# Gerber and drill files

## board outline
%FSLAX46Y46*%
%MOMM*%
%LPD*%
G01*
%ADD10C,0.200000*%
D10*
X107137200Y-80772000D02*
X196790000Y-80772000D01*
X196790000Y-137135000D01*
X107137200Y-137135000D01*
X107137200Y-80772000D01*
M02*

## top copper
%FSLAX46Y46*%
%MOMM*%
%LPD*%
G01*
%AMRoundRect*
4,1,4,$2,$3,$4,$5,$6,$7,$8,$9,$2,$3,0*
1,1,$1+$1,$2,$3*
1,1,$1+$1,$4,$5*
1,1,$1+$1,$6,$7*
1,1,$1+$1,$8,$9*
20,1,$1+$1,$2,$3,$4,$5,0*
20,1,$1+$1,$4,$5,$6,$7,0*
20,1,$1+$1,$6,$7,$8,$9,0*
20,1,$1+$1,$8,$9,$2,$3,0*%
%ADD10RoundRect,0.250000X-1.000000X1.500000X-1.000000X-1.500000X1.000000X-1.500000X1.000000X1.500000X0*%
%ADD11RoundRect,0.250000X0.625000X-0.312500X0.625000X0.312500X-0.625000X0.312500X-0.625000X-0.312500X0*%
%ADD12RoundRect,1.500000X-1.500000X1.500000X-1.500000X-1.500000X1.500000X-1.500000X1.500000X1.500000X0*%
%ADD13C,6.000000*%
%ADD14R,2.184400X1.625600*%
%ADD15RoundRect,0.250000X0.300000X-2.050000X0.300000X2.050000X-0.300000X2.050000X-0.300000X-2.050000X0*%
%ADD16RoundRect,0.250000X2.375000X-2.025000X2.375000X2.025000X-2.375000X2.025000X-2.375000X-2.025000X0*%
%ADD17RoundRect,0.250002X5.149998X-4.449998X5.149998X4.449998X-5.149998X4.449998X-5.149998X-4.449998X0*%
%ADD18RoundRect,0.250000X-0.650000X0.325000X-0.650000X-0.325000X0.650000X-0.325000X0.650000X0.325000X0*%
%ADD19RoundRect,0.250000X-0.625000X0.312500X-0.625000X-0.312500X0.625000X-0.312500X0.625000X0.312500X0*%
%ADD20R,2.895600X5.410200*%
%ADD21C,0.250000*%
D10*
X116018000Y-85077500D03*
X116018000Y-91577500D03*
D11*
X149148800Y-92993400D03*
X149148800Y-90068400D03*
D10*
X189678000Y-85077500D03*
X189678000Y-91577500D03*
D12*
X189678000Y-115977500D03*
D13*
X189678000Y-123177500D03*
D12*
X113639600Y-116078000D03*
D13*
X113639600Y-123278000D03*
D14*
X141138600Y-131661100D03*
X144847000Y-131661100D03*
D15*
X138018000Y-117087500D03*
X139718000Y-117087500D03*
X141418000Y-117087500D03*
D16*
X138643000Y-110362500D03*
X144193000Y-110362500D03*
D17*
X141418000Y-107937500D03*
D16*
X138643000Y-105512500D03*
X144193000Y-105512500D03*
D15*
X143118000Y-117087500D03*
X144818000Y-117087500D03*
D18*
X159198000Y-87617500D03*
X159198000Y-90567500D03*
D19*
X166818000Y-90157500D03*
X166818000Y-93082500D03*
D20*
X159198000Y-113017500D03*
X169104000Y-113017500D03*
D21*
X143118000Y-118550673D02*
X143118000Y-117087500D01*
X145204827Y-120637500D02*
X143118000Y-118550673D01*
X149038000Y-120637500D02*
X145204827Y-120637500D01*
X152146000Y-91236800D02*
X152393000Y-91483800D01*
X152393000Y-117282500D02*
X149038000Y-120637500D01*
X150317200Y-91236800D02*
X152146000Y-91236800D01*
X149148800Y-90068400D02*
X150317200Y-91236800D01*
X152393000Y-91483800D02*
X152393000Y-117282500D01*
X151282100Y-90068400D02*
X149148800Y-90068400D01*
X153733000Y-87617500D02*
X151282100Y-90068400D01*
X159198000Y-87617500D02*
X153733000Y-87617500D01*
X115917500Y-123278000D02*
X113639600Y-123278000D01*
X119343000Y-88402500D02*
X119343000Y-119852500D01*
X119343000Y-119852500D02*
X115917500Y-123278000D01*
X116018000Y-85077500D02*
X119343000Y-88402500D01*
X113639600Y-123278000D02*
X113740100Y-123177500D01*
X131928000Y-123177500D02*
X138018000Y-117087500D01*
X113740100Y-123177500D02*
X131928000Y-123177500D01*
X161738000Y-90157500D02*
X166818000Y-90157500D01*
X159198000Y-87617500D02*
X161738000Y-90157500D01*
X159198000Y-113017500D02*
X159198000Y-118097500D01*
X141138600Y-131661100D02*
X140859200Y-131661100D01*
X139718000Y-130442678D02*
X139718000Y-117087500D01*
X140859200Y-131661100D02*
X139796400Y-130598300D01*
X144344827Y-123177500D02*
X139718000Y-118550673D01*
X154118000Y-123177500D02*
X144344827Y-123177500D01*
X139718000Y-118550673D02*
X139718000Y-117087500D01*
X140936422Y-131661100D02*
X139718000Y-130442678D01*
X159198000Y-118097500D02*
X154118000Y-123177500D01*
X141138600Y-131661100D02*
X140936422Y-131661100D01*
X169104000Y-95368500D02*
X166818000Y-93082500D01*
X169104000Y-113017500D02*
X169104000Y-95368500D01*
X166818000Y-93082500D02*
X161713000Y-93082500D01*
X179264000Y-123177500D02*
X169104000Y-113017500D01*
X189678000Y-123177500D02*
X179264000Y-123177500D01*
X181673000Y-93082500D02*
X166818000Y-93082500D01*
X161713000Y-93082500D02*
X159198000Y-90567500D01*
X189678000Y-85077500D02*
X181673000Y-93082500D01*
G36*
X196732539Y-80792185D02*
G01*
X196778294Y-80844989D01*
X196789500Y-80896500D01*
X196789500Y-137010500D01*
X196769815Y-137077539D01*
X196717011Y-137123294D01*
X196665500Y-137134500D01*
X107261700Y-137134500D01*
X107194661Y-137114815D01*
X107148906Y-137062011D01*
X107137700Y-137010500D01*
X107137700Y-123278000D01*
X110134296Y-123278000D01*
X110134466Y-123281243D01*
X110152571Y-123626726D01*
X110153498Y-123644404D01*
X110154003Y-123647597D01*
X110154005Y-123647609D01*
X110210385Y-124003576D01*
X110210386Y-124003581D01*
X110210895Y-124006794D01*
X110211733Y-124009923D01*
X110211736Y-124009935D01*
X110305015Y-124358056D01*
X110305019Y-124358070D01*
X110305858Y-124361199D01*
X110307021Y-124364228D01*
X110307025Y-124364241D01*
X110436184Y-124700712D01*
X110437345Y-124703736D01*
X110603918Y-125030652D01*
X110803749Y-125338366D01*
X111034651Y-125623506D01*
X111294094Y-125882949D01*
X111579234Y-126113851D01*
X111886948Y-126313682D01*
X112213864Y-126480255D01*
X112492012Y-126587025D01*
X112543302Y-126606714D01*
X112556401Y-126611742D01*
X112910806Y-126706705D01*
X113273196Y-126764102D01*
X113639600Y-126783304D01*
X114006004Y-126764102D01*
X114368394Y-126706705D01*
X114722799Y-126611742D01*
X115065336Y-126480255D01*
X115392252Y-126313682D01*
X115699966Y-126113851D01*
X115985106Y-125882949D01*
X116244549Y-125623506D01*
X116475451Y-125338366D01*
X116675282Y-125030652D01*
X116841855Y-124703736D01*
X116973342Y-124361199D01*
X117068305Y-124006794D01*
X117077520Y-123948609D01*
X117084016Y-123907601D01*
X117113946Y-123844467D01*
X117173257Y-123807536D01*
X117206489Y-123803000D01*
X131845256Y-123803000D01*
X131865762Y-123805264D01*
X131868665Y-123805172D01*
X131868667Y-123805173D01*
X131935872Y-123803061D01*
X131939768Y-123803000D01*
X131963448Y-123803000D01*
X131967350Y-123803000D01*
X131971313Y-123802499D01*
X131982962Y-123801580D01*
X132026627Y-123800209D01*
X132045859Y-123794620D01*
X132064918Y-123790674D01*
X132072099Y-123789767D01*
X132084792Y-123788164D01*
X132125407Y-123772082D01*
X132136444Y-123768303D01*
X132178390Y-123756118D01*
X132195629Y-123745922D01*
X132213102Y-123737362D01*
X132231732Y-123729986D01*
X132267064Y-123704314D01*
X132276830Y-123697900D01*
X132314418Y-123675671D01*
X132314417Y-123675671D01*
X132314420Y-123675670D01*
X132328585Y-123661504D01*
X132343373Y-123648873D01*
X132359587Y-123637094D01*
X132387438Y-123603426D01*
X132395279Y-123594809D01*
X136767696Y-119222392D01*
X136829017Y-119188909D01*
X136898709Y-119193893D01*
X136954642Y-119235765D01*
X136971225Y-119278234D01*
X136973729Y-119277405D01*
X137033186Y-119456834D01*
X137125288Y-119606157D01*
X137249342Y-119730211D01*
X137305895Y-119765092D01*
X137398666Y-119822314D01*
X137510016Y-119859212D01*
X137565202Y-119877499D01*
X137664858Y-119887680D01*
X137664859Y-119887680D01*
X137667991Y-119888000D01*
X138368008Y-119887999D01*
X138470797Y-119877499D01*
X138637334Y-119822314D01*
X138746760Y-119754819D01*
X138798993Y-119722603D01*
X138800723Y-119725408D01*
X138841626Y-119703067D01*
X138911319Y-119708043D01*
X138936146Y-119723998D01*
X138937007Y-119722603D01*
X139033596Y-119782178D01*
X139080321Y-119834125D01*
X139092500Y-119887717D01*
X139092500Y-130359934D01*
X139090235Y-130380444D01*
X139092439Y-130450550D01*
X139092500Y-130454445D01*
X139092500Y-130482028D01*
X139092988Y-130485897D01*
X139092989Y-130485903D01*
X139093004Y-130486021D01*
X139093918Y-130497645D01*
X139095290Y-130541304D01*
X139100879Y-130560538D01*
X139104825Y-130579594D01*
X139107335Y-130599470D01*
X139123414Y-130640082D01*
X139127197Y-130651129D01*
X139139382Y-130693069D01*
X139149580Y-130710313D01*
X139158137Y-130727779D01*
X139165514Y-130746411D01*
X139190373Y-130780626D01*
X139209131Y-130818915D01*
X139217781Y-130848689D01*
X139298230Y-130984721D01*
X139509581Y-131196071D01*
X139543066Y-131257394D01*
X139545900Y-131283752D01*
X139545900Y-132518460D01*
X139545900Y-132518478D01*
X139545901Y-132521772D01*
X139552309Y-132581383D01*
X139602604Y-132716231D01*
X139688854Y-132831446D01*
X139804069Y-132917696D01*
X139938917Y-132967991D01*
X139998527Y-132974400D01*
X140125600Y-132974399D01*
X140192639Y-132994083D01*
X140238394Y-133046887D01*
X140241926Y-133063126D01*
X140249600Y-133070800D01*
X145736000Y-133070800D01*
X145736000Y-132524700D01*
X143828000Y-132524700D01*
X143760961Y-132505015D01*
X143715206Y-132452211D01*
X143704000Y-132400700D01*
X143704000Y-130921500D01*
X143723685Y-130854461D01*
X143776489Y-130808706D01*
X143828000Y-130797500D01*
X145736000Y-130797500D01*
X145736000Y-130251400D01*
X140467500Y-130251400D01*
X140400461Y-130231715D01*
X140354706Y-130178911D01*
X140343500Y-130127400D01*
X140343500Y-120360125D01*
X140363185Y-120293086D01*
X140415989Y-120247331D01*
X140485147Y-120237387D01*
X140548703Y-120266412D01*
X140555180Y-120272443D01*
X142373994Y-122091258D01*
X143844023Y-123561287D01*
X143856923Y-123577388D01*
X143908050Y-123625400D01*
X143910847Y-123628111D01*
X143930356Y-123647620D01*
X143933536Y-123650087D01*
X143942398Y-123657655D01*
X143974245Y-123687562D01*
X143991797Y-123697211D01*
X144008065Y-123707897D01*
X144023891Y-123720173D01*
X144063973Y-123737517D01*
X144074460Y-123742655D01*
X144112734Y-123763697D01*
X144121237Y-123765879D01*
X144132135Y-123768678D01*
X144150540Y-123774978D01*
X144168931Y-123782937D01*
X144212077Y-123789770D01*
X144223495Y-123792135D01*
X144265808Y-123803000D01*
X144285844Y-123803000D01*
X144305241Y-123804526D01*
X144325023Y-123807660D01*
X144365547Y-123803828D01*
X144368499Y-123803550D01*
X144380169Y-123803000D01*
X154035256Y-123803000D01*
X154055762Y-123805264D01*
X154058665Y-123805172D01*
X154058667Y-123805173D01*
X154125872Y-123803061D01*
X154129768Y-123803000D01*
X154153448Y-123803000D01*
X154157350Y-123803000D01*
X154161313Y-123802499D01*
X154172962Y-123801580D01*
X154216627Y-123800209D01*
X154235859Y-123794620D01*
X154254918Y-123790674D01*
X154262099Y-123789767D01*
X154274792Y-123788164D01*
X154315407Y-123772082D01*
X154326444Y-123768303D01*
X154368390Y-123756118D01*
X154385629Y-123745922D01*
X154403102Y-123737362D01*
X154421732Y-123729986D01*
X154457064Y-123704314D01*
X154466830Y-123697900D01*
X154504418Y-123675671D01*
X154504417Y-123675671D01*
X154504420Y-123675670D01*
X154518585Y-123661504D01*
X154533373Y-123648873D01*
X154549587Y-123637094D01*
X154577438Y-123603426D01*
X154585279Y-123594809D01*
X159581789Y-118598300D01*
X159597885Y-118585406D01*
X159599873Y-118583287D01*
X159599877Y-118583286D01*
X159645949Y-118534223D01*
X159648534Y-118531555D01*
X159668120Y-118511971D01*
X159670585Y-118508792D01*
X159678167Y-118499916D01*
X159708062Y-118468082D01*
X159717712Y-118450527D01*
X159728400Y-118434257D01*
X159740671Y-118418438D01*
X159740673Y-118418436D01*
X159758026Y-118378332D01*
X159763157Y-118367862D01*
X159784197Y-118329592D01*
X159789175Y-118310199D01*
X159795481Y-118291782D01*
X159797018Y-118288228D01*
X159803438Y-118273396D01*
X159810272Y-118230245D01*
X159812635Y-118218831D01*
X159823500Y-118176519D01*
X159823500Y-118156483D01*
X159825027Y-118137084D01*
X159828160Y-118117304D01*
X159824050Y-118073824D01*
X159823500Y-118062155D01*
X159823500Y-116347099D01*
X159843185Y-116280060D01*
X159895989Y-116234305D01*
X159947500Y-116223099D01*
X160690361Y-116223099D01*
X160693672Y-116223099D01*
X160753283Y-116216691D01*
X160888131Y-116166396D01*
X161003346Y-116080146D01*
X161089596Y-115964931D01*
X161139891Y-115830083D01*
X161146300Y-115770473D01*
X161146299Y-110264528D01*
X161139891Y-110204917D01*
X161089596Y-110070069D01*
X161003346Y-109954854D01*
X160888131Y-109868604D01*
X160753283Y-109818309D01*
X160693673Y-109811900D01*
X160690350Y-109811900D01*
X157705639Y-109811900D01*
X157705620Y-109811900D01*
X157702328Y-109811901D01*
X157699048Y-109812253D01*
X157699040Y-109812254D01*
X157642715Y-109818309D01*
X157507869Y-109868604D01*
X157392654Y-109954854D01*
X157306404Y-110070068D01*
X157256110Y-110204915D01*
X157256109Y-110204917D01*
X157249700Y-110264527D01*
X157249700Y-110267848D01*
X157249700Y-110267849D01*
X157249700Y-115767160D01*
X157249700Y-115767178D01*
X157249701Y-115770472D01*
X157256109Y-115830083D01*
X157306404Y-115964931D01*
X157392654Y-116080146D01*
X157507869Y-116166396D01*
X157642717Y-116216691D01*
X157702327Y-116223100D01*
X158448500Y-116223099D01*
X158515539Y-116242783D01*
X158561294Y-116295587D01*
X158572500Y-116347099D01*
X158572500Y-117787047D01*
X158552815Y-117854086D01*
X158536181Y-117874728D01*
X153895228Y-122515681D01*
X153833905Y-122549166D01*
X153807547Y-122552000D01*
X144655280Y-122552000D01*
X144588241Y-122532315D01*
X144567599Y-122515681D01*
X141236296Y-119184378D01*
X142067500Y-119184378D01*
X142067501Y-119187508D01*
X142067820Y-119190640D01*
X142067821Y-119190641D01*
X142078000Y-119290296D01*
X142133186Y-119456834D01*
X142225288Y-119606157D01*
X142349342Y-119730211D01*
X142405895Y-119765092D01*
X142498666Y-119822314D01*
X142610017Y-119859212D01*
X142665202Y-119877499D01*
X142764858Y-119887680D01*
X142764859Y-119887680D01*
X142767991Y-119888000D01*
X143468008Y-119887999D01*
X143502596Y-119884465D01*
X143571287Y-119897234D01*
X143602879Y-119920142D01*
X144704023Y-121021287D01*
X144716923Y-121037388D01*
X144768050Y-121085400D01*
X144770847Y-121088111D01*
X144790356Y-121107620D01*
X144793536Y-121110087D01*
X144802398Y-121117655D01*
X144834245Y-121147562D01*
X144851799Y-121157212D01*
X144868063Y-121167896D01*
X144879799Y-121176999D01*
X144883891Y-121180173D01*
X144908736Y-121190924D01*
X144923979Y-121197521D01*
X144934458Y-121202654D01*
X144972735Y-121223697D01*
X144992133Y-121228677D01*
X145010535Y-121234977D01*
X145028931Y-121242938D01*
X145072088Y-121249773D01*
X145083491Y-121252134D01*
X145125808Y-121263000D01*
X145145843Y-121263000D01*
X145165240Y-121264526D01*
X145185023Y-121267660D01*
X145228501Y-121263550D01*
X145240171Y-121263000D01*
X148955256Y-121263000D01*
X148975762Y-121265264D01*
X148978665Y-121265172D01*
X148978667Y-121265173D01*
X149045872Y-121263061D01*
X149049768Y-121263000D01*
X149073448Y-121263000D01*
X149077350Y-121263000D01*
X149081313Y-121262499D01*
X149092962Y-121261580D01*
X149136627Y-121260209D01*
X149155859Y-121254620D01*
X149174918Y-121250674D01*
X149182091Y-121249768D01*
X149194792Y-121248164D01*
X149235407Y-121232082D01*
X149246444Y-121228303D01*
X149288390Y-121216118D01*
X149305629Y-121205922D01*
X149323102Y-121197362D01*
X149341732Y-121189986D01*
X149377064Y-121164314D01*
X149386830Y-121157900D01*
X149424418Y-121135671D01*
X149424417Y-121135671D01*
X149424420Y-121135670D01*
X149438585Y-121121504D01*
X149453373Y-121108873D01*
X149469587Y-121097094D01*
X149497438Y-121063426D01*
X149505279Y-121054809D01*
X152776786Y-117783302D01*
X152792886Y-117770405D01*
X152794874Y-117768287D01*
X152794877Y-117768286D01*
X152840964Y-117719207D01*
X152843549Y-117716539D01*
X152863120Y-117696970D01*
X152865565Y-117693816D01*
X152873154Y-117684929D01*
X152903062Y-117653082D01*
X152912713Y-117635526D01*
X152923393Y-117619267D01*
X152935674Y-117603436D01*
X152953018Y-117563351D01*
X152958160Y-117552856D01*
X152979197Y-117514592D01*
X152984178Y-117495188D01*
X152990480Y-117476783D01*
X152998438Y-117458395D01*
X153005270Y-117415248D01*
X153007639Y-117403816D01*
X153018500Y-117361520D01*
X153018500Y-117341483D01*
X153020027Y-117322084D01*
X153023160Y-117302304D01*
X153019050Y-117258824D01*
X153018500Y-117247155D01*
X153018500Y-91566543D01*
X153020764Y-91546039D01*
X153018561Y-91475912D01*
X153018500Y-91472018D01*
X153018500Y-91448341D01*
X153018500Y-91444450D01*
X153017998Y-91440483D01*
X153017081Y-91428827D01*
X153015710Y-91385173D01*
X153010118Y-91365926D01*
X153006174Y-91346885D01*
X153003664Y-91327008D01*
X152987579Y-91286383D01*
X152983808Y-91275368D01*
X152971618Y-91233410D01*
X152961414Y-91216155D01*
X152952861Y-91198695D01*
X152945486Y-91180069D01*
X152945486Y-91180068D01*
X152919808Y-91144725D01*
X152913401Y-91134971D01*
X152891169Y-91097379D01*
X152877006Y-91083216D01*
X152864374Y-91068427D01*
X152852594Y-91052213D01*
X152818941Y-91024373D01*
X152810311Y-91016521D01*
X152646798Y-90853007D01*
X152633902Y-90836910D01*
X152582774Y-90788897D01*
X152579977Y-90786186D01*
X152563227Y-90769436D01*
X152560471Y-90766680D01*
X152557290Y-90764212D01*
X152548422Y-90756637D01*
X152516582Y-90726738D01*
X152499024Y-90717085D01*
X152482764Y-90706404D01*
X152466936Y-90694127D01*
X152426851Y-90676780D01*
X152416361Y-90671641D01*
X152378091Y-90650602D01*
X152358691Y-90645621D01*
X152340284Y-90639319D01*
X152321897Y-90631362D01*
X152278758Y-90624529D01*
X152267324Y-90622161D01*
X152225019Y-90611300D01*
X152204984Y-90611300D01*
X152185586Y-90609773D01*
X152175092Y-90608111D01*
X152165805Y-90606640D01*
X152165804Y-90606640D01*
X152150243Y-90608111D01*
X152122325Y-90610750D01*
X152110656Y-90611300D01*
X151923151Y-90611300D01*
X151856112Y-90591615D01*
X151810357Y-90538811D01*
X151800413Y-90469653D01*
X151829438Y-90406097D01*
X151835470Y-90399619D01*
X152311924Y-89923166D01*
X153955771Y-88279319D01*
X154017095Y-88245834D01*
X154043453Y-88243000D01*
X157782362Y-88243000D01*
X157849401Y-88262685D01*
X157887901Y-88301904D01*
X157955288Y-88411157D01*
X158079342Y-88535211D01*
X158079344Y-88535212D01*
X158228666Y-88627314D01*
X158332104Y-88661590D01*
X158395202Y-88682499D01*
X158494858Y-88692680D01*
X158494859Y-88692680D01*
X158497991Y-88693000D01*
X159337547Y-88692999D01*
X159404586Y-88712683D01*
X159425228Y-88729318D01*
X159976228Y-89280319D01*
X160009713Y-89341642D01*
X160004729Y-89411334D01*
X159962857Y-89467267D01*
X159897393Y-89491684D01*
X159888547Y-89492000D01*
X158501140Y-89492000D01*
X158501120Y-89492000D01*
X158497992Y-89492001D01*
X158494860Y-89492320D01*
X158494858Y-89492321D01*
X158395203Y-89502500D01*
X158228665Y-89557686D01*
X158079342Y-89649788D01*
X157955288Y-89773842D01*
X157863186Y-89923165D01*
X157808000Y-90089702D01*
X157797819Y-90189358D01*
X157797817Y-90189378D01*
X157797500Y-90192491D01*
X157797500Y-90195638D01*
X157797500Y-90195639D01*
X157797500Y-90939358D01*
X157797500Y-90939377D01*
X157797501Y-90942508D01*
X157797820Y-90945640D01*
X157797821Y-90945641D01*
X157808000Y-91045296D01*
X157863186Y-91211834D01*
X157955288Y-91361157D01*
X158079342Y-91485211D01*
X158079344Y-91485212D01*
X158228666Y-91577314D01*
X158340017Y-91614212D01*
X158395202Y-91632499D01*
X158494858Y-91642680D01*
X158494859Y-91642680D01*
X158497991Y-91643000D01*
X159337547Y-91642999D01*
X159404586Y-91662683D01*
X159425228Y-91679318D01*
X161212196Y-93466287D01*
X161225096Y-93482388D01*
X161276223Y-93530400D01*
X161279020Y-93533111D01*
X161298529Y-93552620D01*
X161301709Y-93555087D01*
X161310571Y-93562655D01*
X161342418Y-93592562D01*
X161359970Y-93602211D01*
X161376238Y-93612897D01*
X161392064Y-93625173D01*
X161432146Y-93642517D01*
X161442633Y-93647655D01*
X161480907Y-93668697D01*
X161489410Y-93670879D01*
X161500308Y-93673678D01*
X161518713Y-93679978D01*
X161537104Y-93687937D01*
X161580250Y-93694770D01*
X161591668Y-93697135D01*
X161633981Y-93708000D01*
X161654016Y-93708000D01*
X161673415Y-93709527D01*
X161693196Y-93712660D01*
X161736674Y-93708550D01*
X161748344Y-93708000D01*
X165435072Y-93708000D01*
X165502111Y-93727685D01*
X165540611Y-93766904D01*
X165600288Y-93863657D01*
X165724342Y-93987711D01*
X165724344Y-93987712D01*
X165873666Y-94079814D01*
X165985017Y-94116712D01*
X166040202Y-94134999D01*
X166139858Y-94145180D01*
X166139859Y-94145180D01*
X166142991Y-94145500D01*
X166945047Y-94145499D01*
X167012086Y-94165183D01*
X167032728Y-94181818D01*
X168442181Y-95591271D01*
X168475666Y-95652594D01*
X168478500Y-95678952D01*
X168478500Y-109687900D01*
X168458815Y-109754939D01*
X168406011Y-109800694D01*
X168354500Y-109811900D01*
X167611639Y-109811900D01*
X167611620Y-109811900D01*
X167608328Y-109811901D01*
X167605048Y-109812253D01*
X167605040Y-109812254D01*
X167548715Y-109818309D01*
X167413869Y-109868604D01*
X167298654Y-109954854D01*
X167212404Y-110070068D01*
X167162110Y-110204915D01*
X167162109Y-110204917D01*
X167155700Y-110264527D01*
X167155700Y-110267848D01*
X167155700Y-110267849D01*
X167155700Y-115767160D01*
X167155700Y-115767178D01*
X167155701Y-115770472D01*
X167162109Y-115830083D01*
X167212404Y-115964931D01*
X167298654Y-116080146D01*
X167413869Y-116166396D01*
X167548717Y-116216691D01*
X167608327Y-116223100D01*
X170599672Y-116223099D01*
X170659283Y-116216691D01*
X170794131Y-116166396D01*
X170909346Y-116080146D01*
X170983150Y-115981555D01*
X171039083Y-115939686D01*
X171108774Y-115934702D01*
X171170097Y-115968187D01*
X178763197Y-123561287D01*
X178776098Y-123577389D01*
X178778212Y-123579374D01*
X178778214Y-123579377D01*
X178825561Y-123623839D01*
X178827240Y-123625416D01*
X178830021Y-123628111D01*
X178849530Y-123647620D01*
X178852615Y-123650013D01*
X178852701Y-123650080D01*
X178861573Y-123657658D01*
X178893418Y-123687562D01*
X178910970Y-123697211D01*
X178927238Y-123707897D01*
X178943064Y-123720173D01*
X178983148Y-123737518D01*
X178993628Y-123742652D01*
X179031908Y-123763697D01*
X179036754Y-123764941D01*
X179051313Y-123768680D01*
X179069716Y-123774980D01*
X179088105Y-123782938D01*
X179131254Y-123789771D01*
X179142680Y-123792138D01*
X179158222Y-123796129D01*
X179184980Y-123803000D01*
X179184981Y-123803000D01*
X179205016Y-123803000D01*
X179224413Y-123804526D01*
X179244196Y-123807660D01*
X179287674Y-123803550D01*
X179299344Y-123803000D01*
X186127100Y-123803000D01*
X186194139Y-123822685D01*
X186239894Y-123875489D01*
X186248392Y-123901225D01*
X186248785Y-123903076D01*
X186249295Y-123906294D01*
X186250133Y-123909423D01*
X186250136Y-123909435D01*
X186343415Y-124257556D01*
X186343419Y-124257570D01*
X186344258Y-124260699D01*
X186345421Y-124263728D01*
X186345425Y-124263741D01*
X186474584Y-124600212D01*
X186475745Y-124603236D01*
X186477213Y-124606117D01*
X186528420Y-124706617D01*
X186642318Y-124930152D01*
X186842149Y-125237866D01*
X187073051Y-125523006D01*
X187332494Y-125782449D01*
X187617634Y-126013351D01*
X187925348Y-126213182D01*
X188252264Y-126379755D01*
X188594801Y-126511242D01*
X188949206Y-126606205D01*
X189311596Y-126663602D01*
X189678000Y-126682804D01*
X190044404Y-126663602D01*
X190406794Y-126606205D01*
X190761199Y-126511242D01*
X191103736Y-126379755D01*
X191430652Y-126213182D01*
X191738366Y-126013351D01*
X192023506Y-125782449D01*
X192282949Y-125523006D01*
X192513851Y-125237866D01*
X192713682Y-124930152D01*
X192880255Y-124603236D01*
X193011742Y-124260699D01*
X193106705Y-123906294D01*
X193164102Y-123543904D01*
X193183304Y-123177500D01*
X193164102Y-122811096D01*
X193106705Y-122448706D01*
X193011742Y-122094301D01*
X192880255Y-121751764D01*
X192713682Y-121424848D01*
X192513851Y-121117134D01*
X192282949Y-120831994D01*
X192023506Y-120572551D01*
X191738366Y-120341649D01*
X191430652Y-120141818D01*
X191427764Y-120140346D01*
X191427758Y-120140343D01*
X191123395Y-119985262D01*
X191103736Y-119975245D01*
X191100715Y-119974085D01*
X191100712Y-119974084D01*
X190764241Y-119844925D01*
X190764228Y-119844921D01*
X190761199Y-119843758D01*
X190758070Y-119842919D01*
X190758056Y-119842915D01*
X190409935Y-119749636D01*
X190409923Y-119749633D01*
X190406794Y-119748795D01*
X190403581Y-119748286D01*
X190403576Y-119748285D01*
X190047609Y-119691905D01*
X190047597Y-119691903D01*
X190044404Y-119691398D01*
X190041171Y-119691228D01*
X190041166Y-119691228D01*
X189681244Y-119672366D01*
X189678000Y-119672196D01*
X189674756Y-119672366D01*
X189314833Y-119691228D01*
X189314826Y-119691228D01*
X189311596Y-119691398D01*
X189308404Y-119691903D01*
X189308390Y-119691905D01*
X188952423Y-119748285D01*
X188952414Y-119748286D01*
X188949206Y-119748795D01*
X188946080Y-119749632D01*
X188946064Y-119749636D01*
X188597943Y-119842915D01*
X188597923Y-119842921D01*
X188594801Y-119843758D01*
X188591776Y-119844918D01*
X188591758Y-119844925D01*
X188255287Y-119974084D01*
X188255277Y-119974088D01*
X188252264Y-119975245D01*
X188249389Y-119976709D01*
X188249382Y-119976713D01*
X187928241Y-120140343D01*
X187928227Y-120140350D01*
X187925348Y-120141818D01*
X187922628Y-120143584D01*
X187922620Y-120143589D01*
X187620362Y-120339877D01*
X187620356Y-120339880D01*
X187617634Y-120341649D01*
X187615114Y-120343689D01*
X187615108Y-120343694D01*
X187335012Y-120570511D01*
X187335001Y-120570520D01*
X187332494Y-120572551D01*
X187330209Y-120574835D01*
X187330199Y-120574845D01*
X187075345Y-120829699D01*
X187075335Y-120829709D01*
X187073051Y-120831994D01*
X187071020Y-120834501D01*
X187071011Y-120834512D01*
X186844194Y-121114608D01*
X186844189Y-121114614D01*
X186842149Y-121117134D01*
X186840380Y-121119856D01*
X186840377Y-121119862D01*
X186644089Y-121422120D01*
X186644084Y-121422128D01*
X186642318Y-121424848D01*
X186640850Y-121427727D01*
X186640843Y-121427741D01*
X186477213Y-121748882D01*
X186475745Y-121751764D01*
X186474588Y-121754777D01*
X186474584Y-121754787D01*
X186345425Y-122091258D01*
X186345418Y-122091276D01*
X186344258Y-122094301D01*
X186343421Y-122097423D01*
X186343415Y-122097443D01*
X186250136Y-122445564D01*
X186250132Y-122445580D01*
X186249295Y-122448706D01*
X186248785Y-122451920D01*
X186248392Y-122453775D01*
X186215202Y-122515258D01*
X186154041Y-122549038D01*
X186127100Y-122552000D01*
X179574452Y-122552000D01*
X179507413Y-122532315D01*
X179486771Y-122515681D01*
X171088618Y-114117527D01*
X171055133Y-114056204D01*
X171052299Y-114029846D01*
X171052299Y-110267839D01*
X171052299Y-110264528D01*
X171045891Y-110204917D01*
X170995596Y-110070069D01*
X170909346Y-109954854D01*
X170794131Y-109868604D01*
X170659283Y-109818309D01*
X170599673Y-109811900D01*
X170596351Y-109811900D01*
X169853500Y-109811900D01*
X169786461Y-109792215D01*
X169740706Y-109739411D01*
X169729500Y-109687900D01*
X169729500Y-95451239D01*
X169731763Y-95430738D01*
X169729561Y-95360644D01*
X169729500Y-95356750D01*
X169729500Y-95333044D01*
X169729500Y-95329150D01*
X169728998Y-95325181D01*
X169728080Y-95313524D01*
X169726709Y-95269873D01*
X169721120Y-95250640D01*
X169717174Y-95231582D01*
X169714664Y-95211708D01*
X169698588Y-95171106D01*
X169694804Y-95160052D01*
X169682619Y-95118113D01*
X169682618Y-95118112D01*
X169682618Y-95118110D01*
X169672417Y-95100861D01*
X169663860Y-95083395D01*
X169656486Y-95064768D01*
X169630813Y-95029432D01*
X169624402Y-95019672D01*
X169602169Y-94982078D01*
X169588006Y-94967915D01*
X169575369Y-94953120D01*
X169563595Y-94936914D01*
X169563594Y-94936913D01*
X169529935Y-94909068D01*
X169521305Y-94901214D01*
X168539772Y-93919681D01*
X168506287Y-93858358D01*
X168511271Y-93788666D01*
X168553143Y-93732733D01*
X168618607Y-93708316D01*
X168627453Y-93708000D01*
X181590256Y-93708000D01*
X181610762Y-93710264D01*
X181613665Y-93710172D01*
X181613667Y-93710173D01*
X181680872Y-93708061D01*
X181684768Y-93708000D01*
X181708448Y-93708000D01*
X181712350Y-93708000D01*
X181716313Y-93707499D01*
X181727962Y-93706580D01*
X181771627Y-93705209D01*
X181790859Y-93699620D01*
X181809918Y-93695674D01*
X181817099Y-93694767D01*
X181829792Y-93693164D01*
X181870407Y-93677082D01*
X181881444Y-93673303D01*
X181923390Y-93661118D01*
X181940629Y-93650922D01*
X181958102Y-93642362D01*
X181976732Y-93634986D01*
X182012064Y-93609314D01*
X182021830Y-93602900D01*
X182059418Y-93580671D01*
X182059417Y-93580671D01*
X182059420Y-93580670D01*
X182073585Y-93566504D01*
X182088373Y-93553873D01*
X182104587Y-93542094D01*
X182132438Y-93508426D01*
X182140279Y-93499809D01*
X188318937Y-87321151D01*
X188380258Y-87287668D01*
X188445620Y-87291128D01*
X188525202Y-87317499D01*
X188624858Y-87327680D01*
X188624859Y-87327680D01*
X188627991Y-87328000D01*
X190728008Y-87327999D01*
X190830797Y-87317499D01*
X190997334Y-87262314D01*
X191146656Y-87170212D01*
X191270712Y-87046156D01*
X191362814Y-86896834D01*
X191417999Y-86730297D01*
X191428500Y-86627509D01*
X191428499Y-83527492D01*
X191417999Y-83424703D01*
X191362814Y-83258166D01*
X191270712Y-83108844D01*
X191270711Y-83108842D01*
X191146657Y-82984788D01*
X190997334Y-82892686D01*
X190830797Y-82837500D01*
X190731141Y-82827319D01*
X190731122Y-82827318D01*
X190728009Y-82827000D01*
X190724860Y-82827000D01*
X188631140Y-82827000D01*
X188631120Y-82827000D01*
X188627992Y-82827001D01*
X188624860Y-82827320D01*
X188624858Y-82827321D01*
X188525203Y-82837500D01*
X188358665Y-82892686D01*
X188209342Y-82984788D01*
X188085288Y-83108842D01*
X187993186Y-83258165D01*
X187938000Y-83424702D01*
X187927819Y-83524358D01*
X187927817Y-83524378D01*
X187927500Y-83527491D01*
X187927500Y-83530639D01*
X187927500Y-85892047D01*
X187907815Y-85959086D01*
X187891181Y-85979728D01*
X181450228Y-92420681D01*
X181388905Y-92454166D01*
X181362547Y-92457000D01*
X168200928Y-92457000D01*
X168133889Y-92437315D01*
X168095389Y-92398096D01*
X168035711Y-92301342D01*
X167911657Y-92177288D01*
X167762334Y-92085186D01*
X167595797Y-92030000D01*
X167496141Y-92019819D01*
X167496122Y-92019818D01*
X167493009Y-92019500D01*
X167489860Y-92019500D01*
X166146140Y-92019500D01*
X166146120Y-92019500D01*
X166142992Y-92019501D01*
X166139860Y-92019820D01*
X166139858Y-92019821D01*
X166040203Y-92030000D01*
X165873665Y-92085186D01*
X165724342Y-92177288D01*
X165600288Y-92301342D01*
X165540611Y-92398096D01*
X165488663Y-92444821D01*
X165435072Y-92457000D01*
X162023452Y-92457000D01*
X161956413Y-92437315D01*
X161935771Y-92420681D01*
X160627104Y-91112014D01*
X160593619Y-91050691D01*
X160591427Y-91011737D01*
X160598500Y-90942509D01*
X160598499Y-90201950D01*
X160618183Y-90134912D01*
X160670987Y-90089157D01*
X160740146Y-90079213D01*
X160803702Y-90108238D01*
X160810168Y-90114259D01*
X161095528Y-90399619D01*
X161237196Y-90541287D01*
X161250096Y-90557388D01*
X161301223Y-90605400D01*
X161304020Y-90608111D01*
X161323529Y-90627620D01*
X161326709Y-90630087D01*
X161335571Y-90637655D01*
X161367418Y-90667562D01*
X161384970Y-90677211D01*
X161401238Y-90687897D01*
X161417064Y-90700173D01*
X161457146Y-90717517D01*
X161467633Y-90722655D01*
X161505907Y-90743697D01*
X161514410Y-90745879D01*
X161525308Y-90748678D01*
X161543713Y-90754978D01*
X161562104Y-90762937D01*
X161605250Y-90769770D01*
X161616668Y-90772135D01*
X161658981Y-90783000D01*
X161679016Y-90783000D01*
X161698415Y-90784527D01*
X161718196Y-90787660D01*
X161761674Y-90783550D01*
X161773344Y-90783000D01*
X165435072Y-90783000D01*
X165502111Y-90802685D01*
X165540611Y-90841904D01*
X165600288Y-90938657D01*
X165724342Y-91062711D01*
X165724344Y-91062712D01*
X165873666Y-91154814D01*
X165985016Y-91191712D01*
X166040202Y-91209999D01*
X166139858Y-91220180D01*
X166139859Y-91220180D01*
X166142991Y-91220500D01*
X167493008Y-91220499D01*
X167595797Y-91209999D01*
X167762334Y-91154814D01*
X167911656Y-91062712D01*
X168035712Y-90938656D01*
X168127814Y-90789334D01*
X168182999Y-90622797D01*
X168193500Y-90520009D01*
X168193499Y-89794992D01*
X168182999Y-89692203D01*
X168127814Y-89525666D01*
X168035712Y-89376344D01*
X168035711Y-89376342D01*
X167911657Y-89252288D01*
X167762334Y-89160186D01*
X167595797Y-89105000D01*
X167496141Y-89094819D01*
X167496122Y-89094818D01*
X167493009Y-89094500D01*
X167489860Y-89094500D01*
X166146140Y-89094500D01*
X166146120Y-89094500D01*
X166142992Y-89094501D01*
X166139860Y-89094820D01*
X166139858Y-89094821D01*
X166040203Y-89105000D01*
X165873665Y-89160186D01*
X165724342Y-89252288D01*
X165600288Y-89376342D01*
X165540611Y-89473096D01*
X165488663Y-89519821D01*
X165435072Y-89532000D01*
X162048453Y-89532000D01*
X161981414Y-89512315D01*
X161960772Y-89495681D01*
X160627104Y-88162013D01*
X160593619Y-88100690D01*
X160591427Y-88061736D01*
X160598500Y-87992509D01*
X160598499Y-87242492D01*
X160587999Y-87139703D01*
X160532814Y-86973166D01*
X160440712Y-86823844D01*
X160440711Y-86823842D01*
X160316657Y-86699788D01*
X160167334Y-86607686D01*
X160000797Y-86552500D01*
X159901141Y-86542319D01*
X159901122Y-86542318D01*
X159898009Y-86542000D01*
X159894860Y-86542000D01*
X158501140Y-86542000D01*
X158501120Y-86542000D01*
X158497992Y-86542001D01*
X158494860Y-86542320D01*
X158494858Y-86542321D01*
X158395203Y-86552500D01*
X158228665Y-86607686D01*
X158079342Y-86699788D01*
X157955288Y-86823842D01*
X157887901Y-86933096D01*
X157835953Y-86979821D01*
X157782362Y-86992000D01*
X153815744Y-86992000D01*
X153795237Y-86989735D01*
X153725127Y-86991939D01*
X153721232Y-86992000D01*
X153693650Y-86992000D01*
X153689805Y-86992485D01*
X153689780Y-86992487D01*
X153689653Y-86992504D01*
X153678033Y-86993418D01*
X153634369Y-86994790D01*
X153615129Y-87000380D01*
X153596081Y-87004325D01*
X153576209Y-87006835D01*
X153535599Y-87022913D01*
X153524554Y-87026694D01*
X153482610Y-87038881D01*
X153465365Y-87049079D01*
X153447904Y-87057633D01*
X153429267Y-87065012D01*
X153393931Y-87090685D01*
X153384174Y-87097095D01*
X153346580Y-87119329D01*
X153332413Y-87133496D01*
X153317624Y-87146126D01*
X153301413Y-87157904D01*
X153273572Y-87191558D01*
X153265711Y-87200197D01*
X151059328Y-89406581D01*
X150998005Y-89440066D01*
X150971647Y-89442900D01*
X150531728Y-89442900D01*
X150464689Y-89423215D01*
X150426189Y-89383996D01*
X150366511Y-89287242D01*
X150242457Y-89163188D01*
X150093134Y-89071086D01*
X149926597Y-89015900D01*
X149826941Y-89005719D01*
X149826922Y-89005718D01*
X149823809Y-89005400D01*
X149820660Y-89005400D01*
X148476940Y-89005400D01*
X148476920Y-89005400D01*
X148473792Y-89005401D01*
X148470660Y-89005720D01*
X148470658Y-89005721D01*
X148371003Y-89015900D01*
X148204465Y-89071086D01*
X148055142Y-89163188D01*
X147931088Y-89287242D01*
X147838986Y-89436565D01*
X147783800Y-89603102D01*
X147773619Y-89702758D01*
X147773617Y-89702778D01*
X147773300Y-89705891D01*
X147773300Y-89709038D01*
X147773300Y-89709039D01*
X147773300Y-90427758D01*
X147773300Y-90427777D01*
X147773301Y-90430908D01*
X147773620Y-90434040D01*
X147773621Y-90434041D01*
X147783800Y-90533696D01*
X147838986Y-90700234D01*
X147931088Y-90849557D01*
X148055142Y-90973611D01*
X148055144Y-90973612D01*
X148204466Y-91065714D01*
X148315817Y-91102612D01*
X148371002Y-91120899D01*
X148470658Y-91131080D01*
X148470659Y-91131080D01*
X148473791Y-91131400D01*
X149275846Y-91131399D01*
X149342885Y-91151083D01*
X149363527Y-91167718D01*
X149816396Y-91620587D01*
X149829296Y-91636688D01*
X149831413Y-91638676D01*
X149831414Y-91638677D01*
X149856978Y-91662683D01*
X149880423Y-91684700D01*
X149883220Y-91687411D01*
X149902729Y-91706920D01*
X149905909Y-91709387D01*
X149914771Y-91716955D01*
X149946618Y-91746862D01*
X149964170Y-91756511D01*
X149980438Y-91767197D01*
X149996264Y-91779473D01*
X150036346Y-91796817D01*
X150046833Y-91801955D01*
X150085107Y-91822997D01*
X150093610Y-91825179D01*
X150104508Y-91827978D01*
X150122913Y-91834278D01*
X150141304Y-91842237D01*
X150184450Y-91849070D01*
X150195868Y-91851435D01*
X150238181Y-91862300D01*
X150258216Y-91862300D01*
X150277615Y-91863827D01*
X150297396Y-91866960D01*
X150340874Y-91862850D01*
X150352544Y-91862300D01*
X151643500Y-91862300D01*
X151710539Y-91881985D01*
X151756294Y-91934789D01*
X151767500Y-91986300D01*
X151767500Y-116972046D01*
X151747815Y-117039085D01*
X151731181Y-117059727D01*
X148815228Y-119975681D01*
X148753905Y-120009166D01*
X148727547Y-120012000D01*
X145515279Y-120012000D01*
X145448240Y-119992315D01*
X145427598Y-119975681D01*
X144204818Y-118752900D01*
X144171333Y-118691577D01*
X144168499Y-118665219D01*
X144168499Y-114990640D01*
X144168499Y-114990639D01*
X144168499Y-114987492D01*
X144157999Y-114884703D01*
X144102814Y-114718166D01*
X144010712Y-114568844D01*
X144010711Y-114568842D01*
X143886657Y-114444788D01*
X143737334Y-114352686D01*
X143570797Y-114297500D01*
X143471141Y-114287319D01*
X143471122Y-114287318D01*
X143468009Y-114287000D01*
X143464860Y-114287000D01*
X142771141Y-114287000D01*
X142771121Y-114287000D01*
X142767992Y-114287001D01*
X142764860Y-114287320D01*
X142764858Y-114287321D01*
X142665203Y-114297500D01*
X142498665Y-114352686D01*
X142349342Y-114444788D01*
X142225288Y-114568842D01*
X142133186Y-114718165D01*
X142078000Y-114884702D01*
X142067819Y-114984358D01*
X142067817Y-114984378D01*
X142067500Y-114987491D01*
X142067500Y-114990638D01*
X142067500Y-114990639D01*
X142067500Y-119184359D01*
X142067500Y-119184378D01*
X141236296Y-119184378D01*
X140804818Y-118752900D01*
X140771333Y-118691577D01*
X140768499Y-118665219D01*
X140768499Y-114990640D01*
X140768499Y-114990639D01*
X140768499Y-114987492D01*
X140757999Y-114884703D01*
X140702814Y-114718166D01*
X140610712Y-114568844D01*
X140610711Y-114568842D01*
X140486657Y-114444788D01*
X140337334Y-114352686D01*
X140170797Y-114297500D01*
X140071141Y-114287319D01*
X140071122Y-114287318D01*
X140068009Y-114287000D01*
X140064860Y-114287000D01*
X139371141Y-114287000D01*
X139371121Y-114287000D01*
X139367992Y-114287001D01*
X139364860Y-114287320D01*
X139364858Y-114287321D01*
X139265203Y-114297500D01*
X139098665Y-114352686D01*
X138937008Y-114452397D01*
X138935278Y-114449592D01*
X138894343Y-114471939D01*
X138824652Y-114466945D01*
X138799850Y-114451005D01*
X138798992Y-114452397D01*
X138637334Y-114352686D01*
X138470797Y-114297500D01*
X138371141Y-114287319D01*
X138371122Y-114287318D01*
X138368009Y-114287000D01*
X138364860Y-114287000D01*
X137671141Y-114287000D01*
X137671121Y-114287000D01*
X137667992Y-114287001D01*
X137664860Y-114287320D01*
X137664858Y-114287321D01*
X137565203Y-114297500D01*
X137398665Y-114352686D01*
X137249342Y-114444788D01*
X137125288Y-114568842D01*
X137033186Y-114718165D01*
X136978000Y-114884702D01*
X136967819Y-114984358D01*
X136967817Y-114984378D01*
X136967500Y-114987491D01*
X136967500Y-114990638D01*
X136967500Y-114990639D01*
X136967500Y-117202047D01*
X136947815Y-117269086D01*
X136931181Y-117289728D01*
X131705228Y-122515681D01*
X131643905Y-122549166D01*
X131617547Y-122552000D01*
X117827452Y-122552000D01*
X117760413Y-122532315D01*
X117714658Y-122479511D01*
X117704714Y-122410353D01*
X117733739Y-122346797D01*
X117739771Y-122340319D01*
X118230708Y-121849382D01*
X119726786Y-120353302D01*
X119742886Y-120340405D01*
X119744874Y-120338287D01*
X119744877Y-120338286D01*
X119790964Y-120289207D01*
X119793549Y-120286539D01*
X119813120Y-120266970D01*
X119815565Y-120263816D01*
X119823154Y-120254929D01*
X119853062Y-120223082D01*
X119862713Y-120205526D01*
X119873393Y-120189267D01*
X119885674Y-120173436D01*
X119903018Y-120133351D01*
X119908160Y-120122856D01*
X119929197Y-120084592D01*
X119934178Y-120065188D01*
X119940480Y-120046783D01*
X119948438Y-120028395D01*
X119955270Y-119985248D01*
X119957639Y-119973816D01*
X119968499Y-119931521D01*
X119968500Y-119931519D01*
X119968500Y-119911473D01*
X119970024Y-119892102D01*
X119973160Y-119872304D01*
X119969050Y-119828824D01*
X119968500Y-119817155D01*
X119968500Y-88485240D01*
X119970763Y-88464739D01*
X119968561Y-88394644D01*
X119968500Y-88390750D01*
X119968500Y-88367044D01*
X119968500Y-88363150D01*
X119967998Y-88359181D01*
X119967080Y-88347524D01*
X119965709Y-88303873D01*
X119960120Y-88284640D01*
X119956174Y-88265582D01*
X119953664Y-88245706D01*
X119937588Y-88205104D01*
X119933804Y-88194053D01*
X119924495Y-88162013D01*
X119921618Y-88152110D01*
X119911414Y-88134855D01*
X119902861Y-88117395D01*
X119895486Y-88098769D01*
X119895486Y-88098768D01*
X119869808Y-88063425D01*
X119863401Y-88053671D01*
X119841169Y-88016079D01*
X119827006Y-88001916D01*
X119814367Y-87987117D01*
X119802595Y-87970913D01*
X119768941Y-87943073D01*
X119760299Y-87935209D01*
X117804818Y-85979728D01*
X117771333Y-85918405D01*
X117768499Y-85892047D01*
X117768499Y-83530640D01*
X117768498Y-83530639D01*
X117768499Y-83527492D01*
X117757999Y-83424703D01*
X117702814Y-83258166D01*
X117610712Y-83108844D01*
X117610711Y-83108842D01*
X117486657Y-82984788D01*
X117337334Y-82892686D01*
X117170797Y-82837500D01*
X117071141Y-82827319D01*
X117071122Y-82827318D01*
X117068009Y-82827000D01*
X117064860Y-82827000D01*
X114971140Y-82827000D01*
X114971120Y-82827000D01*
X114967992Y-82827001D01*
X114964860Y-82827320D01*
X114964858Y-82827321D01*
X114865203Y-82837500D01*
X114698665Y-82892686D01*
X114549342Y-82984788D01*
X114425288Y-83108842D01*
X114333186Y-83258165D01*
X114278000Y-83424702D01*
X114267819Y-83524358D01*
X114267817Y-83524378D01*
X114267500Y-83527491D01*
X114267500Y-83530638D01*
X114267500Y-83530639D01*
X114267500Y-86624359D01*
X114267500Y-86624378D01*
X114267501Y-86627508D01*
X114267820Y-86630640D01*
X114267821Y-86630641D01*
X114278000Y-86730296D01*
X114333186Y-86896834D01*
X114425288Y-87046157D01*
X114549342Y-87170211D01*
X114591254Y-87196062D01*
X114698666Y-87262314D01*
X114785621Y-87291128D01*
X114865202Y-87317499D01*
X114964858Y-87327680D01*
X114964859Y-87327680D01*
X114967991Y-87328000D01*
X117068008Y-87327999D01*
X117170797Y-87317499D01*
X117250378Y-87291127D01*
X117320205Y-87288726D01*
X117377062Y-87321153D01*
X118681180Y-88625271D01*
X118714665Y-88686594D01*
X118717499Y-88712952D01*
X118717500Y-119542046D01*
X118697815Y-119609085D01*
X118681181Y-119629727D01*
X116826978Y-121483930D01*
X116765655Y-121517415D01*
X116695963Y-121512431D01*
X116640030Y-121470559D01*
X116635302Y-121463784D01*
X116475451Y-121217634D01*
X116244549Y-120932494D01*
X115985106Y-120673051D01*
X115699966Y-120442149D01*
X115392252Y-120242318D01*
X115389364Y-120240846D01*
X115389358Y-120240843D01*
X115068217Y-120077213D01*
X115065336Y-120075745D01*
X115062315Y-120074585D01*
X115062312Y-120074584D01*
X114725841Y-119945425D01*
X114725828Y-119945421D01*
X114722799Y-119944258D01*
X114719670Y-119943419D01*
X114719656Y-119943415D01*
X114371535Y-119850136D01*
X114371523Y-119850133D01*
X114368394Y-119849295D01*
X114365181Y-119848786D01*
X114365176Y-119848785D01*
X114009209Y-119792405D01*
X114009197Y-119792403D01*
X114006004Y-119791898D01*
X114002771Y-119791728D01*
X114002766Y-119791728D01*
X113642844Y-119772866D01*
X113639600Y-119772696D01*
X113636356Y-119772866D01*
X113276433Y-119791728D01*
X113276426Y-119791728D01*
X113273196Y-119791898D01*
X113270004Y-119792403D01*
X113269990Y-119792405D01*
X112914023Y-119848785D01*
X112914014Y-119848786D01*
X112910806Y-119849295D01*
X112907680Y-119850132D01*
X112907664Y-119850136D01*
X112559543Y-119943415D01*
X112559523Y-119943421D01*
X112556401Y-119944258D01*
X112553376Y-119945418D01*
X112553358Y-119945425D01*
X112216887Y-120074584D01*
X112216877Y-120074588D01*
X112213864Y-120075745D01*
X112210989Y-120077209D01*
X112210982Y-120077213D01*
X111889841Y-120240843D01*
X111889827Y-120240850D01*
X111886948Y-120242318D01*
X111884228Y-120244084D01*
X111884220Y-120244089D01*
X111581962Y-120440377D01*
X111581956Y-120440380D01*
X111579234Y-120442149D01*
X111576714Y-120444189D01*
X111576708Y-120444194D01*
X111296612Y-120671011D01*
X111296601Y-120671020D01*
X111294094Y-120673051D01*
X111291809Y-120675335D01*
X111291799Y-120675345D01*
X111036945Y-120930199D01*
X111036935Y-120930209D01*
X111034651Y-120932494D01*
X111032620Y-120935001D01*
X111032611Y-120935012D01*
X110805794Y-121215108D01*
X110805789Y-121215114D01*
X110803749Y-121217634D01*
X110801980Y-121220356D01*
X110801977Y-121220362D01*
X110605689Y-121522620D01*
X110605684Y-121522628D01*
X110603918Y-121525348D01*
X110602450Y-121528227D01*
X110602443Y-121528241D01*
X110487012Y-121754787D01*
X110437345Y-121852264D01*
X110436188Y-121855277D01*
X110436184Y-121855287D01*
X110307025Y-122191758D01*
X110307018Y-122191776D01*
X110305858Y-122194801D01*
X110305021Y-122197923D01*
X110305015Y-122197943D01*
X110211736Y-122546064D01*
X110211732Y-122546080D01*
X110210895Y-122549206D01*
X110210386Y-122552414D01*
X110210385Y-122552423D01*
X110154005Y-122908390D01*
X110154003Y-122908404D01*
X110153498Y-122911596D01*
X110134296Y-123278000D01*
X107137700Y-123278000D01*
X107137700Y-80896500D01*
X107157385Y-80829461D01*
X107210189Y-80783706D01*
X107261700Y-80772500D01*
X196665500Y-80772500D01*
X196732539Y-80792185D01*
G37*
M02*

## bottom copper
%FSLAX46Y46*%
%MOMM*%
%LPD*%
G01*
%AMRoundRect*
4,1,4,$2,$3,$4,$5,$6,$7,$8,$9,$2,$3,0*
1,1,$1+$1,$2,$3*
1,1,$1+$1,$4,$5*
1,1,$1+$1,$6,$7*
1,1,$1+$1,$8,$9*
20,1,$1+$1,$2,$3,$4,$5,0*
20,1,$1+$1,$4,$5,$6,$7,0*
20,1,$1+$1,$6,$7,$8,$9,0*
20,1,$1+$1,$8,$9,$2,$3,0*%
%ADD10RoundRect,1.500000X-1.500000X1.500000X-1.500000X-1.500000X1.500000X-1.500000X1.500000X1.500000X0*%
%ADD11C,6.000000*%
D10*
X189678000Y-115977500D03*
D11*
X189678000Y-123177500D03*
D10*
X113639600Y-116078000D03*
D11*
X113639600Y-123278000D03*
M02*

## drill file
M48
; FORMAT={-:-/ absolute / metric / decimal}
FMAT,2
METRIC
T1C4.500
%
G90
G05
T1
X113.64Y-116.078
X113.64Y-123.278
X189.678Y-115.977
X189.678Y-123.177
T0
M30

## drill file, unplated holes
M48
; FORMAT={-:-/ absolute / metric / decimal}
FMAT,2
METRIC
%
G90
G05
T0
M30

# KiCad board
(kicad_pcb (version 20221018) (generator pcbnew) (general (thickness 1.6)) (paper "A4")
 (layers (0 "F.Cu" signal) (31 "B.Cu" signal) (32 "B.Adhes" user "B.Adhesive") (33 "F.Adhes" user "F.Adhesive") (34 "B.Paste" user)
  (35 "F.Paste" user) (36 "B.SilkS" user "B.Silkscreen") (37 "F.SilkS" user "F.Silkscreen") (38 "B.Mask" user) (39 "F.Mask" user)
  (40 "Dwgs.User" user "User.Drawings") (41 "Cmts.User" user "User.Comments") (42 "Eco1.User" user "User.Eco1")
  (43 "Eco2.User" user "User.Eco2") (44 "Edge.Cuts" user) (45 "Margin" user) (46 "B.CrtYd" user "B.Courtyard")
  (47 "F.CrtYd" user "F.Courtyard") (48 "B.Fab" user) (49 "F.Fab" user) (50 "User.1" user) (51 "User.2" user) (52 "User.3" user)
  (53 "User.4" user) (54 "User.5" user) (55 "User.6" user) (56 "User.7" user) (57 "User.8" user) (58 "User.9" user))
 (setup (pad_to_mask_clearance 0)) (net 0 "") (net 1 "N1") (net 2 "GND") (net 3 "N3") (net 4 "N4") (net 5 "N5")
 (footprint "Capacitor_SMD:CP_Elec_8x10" (layer "F.Cu") (at 116.018 88.3275 -90)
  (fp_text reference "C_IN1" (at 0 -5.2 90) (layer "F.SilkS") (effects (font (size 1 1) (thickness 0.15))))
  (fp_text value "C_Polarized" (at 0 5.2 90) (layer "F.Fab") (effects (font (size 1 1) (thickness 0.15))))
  (pad "1" smd roundrect (at -3.25 0 270) (size 3.5 2.5) (layers "F.Cu" "F.Paste" "F.Mask") (roundrect_rratio 0.1) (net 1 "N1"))
  (pad "2" smd roundrect (at 3.25 0 270) (size 3.5 2.5) (layers "F.Cu" "F.Paste" "F.Mask") (roundrect_rratio 0.1) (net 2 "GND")))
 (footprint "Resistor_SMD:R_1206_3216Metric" (layer "F.Cu") (at 149.1488 91.5309 90)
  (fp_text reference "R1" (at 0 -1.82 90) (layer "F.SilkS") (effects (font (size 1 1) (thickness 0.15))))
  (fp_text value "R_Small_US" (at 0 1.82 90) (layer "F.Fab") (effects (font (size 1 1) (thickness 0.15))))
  (pad "1" smd roundrect (at -1.4625 0 90) (size 1.125 1.75) (layers "F.Cu" "F.Paste" "F.Mask") (roundrect_rratio 0.2222222222)
   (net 2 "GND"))
  (pad "2" smd roundrect (at 1.4625 0 90) (size 1.125 1.75) (layers "F.Cu" "F.Paste" "F.Mask") (roundrect_rratio 0.2222222222) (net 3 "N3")))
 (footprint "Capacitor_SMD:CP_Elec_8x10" (layer "F.Cu") (at 189.678 88.3275 -90)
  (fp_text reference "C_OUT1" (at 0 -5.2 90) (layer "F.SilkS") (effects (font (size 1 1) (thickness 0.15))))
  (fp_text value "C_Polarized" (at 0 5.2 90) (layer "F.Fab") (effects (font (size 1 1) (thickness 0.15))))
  (pad "1" smd roundrect (at -3.25 0 270) (size 3.5 2.5) (layers "F.Cu" "F.Paste" "F.Mask") (roundrect_rratio 0.1) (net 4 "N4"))
  (pad "2" smd roundrect (at 3.25 0 270) (size 3.5 2.5) (layers "F.Cu" "F.Paste" "F.Mask") (roundrect_rratio 0.1) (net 2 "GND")))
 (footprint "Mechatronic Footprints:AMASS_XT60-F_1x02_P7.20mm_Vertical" (layer "F.Cu") (at 189.678 115.9775 -90)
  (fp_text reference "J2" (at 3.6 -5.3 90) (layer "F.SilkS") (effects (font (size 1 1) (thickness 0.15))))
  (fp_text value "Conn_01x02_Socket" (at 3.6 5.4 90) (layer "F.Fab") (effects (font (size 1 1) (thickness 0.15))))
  (pad "1" thru_hole roundrect (at 0 0 270) (size 6 6) (drill 4.5) (layers "*.Cu" "*.Mask") (roundrect_rratio 0.25) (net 2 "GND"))
  (pad "2" thru_hole circle (at 7.2 0 270) (size 6 6) (drill 4.5) (layers "*.Cu" "*.Mask") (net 4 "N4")))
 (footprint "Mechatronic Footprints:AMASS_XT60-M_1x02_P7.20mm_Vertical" (layer "F.Cu") (at 113.6396 116.078 -90)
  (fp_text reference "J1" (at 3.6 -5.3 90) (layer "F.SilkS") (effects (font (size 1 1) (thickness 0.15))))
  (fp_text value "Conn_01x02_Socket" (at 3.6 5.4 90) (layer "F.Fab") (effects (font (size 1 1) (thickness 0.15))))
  (pad "1" thru_hole roundrect (at 0 0 270) (size 6 6) (drill 4.5) (layers "*.Cu" "*.Mask") (roundrect_rratio 0.25) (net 2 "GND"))
  (pad "2" thru_hole circle (at 7.2 0 270) (size 6 6) (drill 4.5) (layers "*.Cu" "*.Mask") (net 1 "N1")))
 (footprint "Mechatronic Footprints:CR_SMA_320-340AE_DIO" (layer "F.Cu") (at 142.9928 131.6611)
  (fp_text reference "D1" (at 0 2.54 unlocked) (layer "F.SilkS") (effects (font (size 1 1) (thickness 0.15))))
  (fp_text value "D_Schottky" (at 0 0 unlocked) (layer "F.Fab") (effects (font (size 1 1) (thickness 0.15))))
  (pad "1" smd rect (at -1.8542 0 90) (size 1.6256 2.1844) (layers "F.Cu" "F.Paste" "F.Mask") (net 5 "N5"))
  (pad "2" smd rect (at 1.8542 0 90) (size 1.6256 2.1844) (layers "F.Cu" "F.Paste" "F.Mask") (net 2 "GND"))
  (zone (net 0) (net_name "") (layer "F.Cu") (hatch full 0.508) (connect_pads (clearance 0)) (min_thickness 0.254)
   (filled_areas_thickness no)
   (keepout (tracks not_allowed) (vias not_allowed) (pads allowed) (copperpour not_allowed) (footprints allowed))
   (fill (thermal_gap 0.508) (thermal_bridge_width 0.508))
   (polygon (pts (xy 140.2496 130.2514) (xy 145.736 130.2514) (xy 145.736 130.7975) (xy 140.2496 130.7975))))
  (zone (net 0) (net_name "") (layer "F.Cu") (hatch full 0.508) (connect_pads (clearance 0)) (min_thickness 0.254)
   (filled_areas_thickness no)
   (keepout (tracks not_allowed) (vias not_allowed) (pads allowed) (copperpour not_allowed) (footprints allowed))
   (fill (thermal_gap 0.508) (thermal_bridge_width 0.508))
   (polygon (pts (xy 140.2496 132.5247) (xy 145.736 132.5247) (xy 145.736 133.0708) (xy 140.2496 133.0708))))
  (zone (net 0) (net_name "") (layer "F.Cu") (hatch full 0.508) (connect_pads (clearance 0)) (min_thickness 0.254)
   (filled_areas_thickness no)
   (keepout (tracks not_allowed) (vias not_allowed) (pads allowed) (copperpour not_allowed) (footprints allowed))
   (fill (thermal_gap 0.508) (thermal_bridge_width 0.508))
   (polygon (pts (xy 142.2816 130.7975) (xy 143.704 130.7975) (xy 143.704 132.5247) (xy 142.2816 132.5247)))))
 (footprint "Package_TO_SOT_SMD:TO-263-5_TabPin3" (layer "F.Cu") (at 141.418 109.4375 90)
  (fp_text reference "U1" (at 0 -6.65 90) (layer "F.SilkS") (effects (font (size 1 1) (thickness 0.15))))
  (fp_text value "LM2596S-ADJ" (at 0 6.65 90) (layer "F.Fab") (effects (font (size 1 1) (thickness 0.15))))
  (pad "1" smd roundrect (at -7.65 -3.4 90) (size 4.6 1.1) (layers "F.Cu" "F.Paste" "F.Mask") (roundrect_rratio 0.2272727273) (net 1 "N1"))
  (pad "2" smd roundrect (at -7.65 -1.7 90) (size 4.6 1.1) (layers "F.Cu" "F.Paste" "F.Mask") (roundrect_rratio 0.2272727273) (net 5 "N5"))
  (pad "3" smd roundrect (at -7.65 0 90) (size 4.6 1.1) (layers "F.Cu" "F.Paste" "F.Mask") (roundrect_rratio 0.2272727273) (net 2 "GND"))
  (pad "3" smd roundrect (at -0.925 -2.775 90) (size 4.55 5.25) (layers "F.Cu" "F.Paste") (roundrect_rratio 0.05494505495) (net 2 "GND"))
  (pad "3" smd roundrect (at -0.925 2.775 90) (size 4.55 5.25) (layers "F.Cu" "F.Paste") (roundrect_rratio 0.05494505495) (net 2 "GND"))
  (pad "3" smd roundrect (at 1.5 0 90) (size 9.4 10.8) (layers "F.Cu" "F.Mask") (roundrect_rratio 0.02659595745) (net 2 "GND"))
  (pad "3" smd roundrect (at 3.925 -2.775 90) (size 4.55 5.25) (layers "F.Cu" "F.Paste") (roundrect_rratio 0.05494505495) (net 2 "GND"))
  (pad "3" smd roundrect (at 3.925 2.775 90) (size 4.55 5.25) (layers "F.Cu" "F.Paste") (roundrect_rratio 0.05494505495) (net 2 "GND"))
  (pad "4" smd roundrect (at -7.65 1.7 90) (size 4.6 1.1) (layers "F.Cu" "F.Paste" "F.Mask") (roundrect_rratio 0.2272727273) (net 3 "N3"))
  (pad "5" smd roundrect (at -7.65 3.4 90) (size 4.6 1.1) (layers "F.Cu" "F.Paste" "F.Mask") (roundrect_rratio 0.2272727273) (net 2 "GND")))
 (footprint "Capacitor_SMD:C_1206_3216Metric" (layer "F.Cu") (at 159.198 89.0925 -90)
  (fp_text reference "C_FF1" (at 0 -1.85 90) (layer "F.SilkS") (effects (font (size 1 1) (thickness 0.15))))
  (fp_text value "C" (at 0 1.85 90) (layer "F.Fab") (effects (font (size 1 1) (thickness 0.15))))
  (pad "1" smd roundrect (at -1.475 0 270) (size 1.15 1.8) (layers "F.Cu" "F.Paste" "F.Mask") (roundrect_rratio 0.2173913043) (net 3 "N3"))
  (pad "2" smd roundrect (at 1.475 0 270) (size 1.15 1.8) (layers "F.Cu" "F.Paste" "F.Mask") (roundrect_rratio 0.2173913043) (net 4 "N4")))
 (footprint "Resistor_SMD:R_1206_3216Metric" (layer "F.Cu") (at 166.818 91.62 -90)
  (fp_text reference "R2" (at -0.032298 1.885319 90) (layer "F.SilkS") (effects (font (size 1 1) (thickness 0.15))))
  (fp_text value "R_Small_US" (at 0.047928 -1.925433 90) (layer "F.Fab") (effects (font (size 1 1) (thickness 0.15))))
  (pad "1" smd roundrect (at -1.4625 0 270) (size 1.125 1.75) (layers "F.Cu" "F.Paste" "F.Mask") (roundrect_rratio 0.2222222222)
   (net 3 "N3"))
  (pad "2" smd roundrect (at 1.4625 0 270) (size 1.125 1.75) (layers "F.Cu" "F.Paste" "F.Mask") (roundrect_rratio 0.2222222222) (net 4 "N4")))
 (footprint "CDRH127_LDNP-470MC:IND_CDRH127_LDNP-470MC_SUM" (layer "F.Cu") (at 164.151 113.0175)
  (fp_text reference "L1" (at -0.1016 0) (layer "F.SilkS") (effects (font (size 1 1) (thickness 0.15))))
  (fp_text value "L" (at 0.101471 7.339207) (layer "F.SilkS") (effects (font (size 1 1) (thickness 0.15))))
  (pad "1" smd rect (at -4.953 0) (size 2.8956 5.4102) (layers "F.Cu" "F.Paste" "F.Mask") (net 5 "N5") (solder_mask_margin 0.102))
  (pad "2" smd rect (at 4.953 0) (size 2.8956 5.4102) (layers "F.Cu" "F.Paste" "F.Mask") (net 4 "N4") (solder_mask_margin 0.102)))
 (gr_rect (start 107.1372 80.772) (end 196.79 137.135) (stroke (width 0.2) (type default)) (fill none) (layer "Edge.Cuts"))
 (segment (start 145.204827 120.6375) (end 143.118 118.550673) (width 0.25) (layer "F.Cu") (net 3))
 (segment (start 159.198 87.6175) (end 153.733 87.6175) (width 0.25) (layer "F.Cu") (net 3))
 (segment (start 149.038 120.6375) (end 145.204827 120.6375) (width 0.25) (layer "F.Cu") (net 3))
 (segment (start 161.738 90.1575) (end 166.818 90.1575) (width 0.25) (layer "F.Cu") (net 3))
 (segment (start 143.118 118.550673) (end 143.118 117.0875) (width 0.25) (layer "F.Cu") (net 3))
 (segment (start 152.393 91.4838) (end 152.393 117.2825) (width 0.25) (layer "F.Cu") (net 3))
 (segment (start 152.393 117.2825) (end 149.038 120.6375) (width 0.25) (layer "F.Cu") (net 3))
 (segment (start 153.733 87.6175) (end 151.2821 90.0684) (width 0.25) (layer "F.Cu") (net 3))
 (segment (start 152.146 91.2368) (end 152.393 91.4838) (width 0.25) (layer "F.Cu") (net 3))
 (segment (start 159.198 87.6175) (end 161.738 90.1575) (width 0.25) (layer "F.Cu") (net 3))
 (segment (start 151.2821 90.0684) (end 149.1488 90.0684) (width 0.25) (layer "F.Cu") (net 3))
 (segment (start 149.1488 90.0684) (end 150.3172 91.2368) (width 0.25) (layer "F.Cu") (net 3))
 (segment (start 150.3172 91.2368) (end 152.146 91.2368) (width 0.25) (layer "F.Cu") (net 3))
 (segment (start 159.198 113.0175) (end 159.198 118.0975) (width 0.25) (layer "F.Cu") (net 5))
 (segment (start 141.1386 131.6611) (end 140.8592 131.6611) (width 0.25) (layer "F.Cu") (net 5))
 (segment (start 139.718 130.442678) (end 139.718 117.0875) (width 0.25) (layer "F.Cu") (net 5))
 (segment (start 140.8592 131.6611) (end 139.7964 130.5983) (width 0.25) (layer "F.Cu") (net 5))
 (segment (start 144.344827 123.1775) (end 139.718 118.550673) (width 0.25) (layer "F.Cu") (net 5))
 (segment (start 154.118 123.1775) (end 144.344827 123.1775) (width 0.25) (layer "F.Cu") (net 5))
 (segment (start 139.718 118.550673) (end 139.718 117.0875) (width 0.25) (layer "F.Cu") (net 5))
 (segment (start 140.936422 131.6611) (end 139.718 130.442678) (width 0.25) (layer "F.Cu") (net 5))
 (segment (start 159.198 118.0975) (end 154.118 123.1775) (width 0.25) (layer "F.Cu") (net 5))
 (segment (start 141.1386 131.6611) (end 140.936422 131.6611) (width 0.25) (layer "F.Cu") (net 5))
 (segment (start 169.104 95.3685) (end 166.818 93.0825) (width 0.25) (layer "F.Cu") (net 4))
 (segment (start 169.104 113.0175) (end 169.104 95.3685) (width 0.25) (layer "F.Cu") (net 4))
 (segment (start 166.818 93.0825) (end 161.713 93.0825) (width 0.25) (layer "F.Cu") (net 4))
 (segment (start 179.264 123.1775) (end 169.104 113.0175) (width 0.25) (layer "F.Cu") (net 4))
 (segment (start 189.678 123.1775) (end 179.264 123.1775) (width 0.25) (layer "F.Cu") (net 4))
 (segment (start 181.673 93.0825) (end 166.818 93.0825) (width 0.25) (layer "F.Cu") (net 4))
 (segment (start 161.713 93.0825) (end 159.198 90.5675) (width 0.25) (layer "F.Cu") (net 4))
 (segment (start 189.678 85.0775) (end 181.673 93.0825) (width 0.25) (layer "F.Cu") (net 4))
 (segment (start 116.018 85.0775) (end 119.343 88.4025) (width 0.25) (layer "F.Cu") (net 1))
 (segment (start 113.7401 123.1775) (end 131.928 123.1775) (width 0.25) (layer "F.Cu") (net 1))
 (segment (start 119.343 119.8525) (end 115.9175 123.278) (width 0.25) (layer "F.Cu") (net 1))
 (segment (start 119.343 88.4025) (end 119.343 119.8525) (width 0.25) (layer "F.Cu") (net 1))
 (segment (start 115.9175 123.278) (end 113.6396 123.278) (width 0.25) (layer "F.Cu") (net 1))
 (segment (start 131.928 123.1775) (end 138.018 117.0875) (width 0.25) (layer "F.Cu") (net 1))
 (segment (start 113.6396 123.278) (end 113.7401 123.1775) (width 0.25) (layer "F.Cu") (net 1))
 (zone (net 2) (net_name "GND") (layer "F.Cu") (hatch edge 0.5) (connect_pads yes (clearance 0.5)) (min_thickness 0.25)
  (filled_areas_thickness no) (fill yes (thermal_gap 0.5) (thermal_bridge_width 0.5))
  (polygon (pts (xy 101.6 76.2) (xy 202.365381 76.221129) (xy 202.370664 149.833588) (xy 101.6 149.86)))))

